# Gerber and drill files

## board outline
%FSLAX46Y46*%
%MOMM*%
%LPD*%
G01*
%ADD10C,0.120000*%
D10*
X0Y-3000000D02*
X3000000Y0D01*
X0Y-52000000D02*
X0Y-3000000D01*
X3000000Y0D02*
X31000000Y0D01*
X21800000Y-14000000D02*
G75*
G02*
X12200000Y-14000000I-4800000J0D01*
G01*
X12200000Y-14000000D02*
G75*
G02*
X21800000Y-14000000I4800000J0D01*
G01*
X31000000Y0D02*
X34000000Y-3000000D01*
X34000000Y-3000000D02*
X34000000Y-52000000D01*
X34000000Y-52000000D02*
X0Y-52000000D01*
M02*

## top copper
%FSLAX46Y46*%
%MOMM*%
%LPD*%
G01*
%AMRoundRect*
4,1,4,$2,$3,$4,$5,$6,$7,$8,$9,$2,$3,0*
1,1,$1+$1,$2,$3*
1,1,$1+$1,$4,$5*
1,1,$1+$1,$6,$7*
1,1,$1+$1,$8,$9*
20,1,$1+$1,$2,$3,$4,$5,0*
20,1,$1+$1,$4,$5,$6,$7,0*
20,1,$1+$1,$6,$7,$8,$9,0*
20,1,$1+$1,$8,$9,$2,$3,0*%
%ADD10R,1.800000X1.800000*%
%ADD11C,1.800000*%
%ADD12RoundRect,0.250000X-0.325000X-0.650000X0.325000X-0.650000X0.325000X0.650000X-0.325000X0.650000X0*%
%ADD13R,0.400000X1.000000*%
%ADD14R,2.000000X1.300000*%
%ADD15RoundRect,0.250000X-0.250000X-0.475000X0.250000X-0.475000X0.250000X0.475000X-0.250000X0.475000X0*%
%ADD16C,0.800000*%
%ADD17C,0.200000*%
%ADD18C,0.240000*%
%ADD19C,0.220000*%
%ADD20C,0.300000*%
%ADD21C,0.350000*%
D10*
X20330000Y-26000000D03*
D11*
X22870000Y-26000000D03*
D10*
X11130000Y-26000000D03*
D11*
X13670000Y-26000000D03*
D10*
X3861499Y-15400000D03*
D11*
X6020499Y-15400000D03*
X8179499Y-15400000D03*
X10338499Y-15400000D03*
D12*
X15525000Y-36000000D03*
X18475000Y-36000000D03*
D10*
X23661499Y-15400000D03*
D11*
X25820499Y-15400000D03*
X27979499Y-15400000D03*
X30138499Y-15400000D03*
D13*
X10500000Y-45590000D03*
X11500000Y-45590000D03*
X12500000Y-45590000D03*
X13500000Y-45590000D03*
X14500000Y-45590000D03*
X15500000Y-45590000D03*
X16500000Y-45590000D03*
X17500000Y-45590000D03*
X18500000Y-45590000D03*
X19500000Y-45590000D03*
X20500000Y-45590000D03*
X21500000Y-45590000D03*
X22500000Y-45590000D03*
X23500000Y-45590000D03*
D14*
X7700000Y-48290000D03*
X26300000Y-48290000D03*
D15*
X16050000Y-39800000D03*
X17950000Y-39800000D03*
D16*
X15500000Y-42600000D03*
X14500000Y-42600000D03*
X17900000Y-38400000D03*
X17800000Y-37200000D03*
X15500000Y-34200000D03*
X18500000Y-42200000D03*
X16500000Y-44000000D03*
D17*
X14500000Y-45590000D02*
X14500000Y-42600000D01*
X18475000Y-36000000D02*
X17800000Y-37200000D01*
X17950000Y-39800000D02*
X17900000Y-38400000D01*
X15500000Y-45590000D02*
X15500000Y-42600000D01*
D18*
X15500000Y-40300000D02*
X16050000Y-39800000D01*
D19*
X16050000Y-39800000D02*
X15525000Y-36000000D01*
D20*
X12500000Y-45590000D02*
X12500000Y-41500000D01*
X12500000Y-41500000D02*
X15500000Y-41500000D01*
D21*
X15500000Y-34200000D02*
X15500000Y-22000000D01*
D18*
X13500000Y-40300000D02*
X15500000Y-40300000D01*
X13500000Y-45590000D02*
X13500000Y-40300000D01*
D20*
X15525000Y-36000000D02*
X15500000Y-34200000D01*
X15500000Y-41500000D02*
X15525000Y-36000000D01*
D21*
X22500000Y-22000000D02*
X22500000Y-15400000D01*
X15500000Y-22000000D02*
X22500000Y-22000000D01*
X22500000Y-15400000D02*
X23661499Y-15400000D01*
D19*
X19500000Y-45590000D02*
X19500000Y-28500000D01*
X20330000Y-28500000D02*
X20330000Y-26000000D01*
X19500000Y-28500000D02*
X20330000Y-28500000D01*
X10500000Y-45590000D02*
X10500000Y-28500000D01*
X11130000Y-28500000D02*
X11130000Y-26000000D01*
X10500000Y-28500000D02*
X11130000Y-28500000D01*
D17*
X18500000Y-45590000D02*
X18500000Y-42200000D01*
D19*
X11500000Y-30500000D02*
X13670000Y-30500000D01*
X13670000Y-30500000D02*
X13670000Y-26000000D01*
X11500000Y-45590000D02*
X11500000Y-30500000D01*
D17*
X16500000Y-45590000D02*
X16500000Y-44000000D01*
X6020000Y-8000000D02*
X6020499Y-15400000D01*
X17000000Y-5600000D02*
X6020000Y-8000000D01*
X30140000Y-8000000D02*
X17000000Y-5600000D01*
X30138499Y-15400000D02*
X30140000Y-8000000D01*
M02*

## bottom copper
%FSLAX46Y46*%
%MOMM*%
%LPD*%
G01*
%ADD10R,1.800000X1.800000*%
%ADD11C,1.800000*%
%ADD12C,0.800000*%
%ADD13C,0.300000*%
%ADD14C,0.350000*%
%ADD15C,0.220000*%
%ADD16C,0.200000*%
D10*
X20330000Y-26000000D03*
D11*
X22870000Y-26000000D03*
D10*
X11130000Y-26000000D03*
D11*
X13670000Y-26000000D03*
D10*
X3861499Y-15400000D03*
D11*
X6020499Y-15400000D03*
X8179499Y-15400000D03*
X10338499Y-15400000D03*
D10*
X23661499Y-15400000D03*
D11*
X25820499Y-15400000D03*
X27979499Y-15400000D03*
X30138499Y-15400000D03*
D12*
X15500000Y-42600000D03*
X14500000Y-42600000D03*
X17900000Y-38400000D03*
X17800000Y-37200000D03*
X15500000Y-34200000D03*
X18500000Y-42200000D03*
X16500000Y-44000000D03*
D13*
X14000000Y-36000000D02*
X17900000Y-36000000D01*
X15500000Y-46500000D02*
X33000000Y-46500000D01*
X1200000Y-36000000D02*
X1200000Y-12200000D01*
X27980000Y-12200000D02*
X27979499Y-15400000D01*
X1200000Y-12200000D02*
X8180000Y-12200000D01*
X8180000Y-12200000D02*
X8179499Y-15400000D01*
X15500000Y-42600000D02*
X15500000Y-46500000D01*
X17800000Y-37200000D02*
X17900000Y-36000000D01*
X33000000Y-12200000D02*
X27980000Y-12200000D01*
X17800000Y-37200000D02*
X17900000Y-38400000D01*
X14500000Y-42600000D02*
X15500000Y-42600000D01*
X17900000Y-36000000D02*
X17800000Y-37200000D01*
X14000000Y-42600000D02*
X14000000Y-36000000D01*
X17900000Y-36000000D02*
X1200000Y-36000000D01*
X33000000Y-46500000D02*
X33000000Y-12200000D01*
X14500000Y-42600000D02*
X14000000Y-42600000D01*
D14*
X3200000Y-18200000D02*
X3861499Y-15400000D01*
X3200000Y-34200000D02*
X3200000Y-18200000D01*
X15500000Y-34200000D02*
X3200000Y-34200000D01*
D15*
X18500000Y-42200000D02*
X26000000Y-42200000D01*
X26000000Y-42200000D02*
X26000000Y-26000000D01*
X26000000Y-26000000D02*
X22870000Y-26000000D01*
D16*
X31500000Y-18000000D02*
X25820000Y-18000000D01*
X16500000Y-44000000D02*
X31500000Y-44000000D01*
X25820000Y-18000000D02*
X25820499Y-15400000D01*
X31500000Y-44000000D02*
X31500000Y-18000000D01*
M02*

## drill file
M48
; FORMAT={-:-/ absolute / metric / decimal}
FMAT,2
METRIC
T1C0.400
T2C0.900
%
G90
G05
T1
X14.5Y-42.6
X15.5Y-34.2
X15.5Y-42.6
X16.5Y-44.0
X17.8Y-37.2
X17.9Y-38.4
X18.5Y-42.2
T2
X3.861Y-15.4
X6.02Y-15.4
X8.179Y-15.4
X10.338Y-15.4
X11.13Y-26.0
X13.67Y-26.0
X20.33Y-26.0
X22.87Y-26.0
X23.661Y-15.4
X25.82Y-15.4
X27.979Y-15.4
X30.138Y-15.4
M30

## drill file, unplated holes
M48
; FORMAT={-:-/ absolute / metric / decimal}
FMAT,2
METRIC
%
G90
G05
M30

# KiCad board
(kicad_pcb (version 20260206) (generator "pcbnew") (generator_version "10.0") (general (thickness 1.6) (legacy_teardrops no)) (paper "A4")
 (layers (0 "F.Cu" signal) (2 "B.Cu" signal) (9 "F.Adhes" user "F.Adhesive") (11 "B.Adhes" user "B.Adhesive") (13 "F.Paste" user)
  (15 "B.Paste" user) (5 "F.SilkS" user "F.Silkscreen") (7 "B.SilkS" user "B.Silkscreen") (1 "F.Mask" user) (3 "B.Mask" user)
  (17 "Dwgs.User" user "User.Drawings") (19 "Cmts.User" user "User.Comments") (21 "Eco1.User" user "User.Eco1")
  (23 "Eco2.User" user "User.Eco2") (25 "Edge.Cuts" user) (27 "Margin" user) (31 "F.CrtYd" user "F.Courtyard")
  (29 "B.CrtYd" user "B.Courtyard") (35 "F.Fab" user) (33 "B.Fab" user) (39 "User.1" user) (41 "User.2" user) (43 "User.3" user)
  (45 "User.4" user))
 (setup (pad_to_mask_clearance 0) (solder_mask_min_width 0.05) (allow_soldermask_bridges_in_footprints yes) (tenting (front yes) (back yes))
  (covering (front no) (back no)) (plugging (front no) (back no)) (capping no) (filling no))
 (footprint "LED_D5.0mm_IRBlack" (layer "F.Cu") (at 20.33 26)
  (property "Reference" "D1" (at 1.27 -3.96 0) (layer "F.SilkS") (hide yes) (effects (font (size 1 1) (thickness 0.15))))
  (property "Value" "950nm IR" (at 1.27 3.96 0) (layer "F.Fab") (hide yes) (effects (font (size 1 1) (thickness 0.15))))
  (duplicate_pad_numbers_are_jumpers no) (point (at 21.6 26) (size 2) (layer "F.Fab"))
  (pad "1" thru_hole rect (at 0 0) (size 1.8 1.8) (drill 0.9) (layers "*.Cu" "*.Mask") (remove_unused_layers no) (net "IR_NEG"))
  (pad "2" thru_hole circle (at 2.54 0) (size 1.8 1.8) (drill 0.9) (layers "*.Cu" "*.Mask") (remove_unused_layers no) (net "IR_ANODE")))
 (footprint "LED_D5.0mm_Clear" (layer "F.Cu") (at 11.13 26)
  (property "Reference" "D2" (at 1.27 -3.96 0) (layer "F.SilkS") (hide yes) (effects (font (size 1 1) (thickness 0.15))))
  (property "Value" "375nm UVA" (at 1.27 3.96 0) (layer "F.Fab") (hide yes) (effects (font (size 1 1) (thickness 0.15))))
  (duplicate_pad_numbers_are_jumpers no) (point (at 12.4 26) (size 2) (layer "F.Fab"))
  (pad "1" thru_hole rect (at 0 0) (size 1.8 1.8) (drill 0.9) (layers "*.Cu" "*.Mask") (remove_unused_layers no) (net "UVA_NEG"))
  (pad "2" thru_hole circle (at 2.54 0) (size 1.8 1.8) (drill 0.9) (layers "*.Cu" "*.Mask") (remove_unused_layers no) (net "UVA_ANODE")))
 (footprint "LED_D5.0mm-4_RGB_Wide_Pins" (layer "F.Cu") (at 3.861499 15.4)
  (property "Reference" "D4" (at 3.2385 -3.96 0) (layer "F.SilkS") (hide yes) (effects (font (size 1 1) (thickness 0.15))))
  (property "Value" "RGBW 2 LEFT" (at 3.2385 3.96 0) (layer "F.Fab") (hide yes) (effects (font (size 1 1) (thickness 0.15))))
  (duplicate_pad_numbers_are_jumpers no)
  (pad "1" thru_hole rect (at 0 0) (size 1.8 1.8) (drill 0.9) (layers "*.Cu" "*.Mask") (remove_unused_layers no) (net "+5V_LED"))
  (pad "2" thru_hole circle (at 2.159 0) (size 1.8 1.8) (drill 0.9) (layers "*.Cu" "*.Mask") (remove_unused_layers no) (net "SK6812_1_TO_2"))
  (pad "3" thru_hole circle (at 4.318 0) (size 1.8 1.8) (drill 0.9) (layers "*.Cu" "*.Mask") (remove_unused_layers no) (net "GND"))
  (pad "4" thru_hole circle (at 6.477 0) (size 1.8 1.8) (drill 0.9) (layers "*.Cu" "*.Mask") (remove_unused_layers no)))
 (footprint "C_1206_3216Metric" (layer "F.Cu") (at 17 36)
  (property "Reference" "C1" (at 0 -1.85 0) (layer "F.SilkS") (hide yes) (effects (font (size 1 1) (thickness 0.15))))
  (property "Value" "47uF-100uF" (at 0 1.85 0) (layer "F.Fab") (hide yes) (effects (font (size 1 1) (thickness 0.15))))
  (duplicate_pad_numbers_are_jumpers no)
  (pad "1" smd roundrect (at -1.475 0) (size 1.15 1.8) (layers "F.Cu" "F.Mask" "F.Paste") (roundrect_rratio 0.217391) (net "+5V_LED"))
  (pad "2" smd roundrect (at 1.475 0) (size 1.15 1.8) (layers "F.Cu" "F.Mask" "F.Paste") (roundrect_rratio 0.217391) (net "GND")))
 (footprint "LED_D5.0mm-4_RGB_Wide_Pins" (layer "F.Cu") (at 23.661499 15.4)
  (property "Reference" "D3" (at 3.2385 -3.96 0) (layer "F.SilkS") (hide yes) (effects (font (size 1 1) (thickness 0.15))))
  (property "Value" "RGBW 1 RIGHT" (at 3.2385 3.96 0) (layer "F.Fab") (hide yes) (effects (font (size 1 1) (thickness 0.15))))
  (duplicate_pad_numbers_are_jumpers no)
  (pad "1" thru_hole rect (at 0 0) (size 1.8 1.8) (drill 0.9) (layers "*.Cu" "*.Mask") (remove_unused_layers no) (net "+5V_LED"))
  (pad "2" thru_hole circle (at 2.159 0) (size 1.8 1.8) (drill 0.9) (layers "*.Cu" "*.Mask") (remove_unused_layers no) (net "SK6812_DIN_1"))
  (pad "3" thru_hole circle (at 4.318 0) (size 1.8 1.8) (drill 0.9) (layers "*.Cu" "*.Mask") (remove_unused_layers no) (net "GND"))
  (pad "4" thru_hole circle (at 6.477 0) (size 1.8 1.8) (drill 0.9) (layers "*.Cu" "*.Mask") (remove_unused_layers no) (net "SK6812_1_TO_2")))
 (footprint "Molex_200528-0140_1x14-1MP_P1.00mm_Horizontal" (layer "F.Cu") (at 17 46.5)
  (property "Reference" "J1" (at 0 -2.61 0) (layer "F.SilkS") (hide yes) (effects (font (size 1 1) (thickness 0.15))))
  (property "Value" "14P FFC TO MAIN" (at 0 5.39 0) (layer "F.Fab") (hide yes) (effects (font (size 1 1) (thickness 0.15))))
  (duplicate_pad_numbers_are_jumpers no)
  (pad "1" smd rect (at -6.5 -0.91) (size 0.4 1) (layers "F.Cu" "F.Mask" "F.Paste") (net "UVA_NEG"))
  (pad "2" smd rect (at -5.5 -0.91) (size 0.4 1) (layers "F.Cu" "F.Mask" "F.Paste") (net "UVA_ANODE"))
  (pad "3" smd rect (at -4.5 -0.91) (size 0.4 1) (layers "F.Cu" "F.Mask" "F.Paste") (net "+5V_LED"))
  (pad "4" smd rect (at -3.5 -0.91) (size 0.4 1) (layers "F.Cu" "F.Mask" "F.Paste") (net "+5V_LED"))
  (pad "5" smd rect (at -2.5 -0.91) (size 0.4 1) (layers "F.Cu" "F.Mask" "F.Paste") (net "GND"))
  (pad "6" smd rect (at -1.5 -0.91) (size 0.4 1) (layers "F.Cu" "F.Mask" "F.Paste") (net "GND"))
  (pad "7" smd rect (at -0.5 -0.91) (size 0.4 1) (layers "F.Cu" "F.Mask" "F.Paste") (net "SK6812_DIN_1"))
  (pad "8" smd rect (at 0.5 -0.91) (size 0.4 1) (layers "F.Cu" "F.Mask" "F.Paste"))
  (pad "9" smd rect (at 1.5 -0.91) (size 0.4 1) (layers "F.Cu" "F.Mask" "F.Paste") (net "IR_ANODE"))
  (pad "10" smd rect (at 2.5 -0.91) (size 0.4 1) (layers "F.Cu" "F.Mask" "F.Paste") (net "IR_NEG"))
  (pad "11" smd rect (at 3.5 -0.91) (size 0.4 1) (layers "F.Cu" "F.Mask" "F.Paste"))
  (pad "12" smd rect (at 4.5 -0.91) (size 0.4 1) (layers "F.Cu" "F.Mask" "F.Paste"))
  (pad "13" smd rect (at 5.5 -0.91) (size 0.4 1) (layers "F.Cu" "F.Mask" "F.Paste"))
  (pad "14" smd rect (at 6.5 -0.91) (size 0.4 1) (layers "F.Cu" "F.Mask" "F.Paste"))
  (pad "MP" smd rect (at -9.3 1.79) (size 2 1.3) (layers "F.Cu" "F.Mask" "F.Paste"))
  (pad "MP" smd rect (at 9.3 1.79) (size 2 1.3) (layers "F.Cu" "F.Mask" "F.Paste")))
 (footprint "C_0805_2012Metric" (layer "F.Cu") (at 17 39.8)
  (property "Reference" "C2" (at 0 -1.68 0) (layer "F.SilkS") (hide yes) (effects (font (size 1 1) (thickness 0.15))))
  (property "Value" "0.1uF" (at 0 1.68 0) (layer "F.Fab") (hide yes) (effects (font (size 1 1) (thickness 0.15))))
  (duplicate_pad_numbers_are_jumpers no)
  (pad "1" smd roundrect (at -0.95 0) (size 1 1.45) (layers "F.Cu" "F.Mask" "F.Paste") (roundrect_rratio 0.25) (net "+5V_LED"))
  (pad "2" smd roundrect (at 0.95 0) (size 1 1.45) (layers "F.Cu" "F.Mask" "F.Paste") (roundrect_rratio 0.25) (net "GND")))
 (gr_line (start 0 3) (end 3 0) (stroke (width 0.12) (type default)) (layer "Edge.Cuts"))
 (gr_line (start 0 52) (end 0 3) (stroke (width 0.12) (type default)) (layer "Edge.Cuts"))
 (gr_line (start 3 0) (end 31 0) (stroke (width 0.12) (type default)) (layer "Edge.Cuts"))
 (gr_circle (center 17 14) (end 21.8 14) (stroke (width 0.12) (type default)) (fill no) (layer "Edge.Cuts"))
 (gr_line (start 31 0) (end 34 3) (stroke (width 0.12) (type default)) (layer "Edge.Cuts"))
 (gr_line (start 34 3) (end 34 52) (stroke (width 0.12) (type default)) (layer "Edge.Cuts"))
 (gr_line (start 34 52) (end 0 52) (stroke (width 0.12) (type default)) (layer "Edge.Cuts"))
 (segment (start 14.5 45.59) (end 14.5 42.6) (width 0.2) (layer "F.Cu") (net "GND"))
 (segment (start 18.475 36) (end 17.8 37.2) (width 0.2) (layer "F.Cu") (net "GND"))
 (segment (start 17.95 39.8) (end 17.9 38.4) (width 0.2) (layer "F.Cu") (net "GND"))
 (segment (start 15.5 45.59) (end 15.5 42.6) (width 0.2) (layer "F.Cu") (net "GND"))
 (via (at 15.5 42.6) (size 0.8) (drill 0.4) (layers "F.Cu" "B.Cu") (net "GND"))
 (via (at 14.5 42.6) (size 0.8) (drill 0.4) (layers "F.Cu" "B.Cu") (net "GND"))
 (via (at 17.9 38.4) (size 0.8) (drill 0.4) (layers "F.Cu" "B.Cu") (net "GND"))
 (via (at 17.8 37.2) (size 0.8) (drill 0.4) (layers "F.Cu" "B.Cu") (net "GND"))
 (segment (start 14 36) (end 17.9 36) (width 0.3) (layer "B.Cu") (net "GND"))
 (segment (start 15.5 46.5) (end 33 46.5) (width 0.3) (layer "B.Cu") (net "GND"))
 (segment (start 1.2 36) (end 1.2 12.2) (width 0.3) (layer "B.Cu") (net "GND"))
 (segment (start 27.98 12.2) (end 27.979499 15.4) (width 0.3) (layer "B.Cu") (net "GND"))
 (segment (start 1.2 12.2) (end 8.18 12.2) (width 0.3) (layer "B.Cu") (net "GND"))
 (segment (start 8.18 12.2) (end 8.179499 15.4) (width 0.3) (layer "B.Cu") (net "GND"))
 (segment (start 15.5 42.6) (end 15.5 46.5) (width 0.3) (layer "B.Cu") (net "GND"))
 (segment (start 17.8 37.2) (end 17.9 36) (width 0.3) (layer "B.Cu") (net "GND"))
 (segment (start 33 12.2) (end 27.98 12.2) (width 0.3) (layer "B.Cu") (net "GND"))
 (segment (start 17.8 37.2) (end 17.9 38.4) (width 0.3) (layer "B.Cu") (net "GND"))
 (segment (start 14.5 42.6) (end 15.5 42.6) (width 0.3) (layer "B.Cu") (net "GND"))
 (segment (start 17.9 36) (end 17.8 37.2) (width 0.3) (layer "B.Cu") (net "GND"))
 (segment (start 14 42.6) (end 14 36) (width 0.3) (layer "B.Cu") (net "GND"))
 (segment (start 17.9 36) (end 1.2 36) (width 0.3) (layer "B.Cu") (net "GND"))
 (segment (start 33 46.5) (end 33 12.2) (width 0.3) (layer "B.Cu") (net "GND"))
 (segment (start 14.5 42.6) (end 14 42.6) (width 0.3) (layer "B.Cu") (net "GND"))
 (segment (start 15.5 40.3) (end 16.05 39.8) (width 0.24) (layer "F.Cu") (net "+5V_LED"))
 (segment (start 16.05 39.8) (end 15.525 36) (width 0.22) (layer "F.Cu") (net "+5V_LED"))
 (segment (start 12.5 45.59) (end 12.5 41.5) (width 0.3) (layer "F.Cu") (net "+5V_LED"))
 (segment (start 12.5 41.5) (end 15.5 41.5) (width 0.3) (layer "F.Cu") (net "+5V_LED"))
 (segment (start 15.5 34.2) (end 15.5 22) (width 0.35) (layer "F.Cu") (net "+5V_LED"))
 (segment (start 13.5 40.3) (end 15.5 40.3) (width 0.24) (layer "F.Cu") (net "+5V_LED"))
 (segment (start 13.5 45.59) (end 13.5 40.3) (width 0.24) (layer "F.Cu") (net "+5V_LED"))
 (segment (start 15.525 36) (end 15.5 34.2) (width 0.3) (layer "F.Cu") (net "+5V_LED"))
 (segment (start 15.5 41.5) (end 15.525 36) (width 0.3) (layer "F.Cu") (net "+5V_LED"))
 (segment (start 22.5 22) (end 22.5 15.4) (width 0.35) (layer "F.Cu") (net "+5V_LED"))
 (segment (start 15.5 22) (end 22.5 22) (width 0.35) (layer "F.Cu") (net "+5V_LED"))
 (segment (start 22.5 15.4) (end 23.661499 15.4) (width 0.35) (layer "F.Cu") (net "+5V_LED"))
 (via (at 15.5 34.2) (size 0.8) (drill 0.4) (layers "F.Cu" "B.Cu") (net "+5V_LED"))
 (segment (start 3.2 18.2) (end 3.861499 15.4) (width 0.35) (layer "B.Cu") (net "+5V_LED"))
 (segment (start 3.2 34.2) (end 3.2 18.2) (width 0.35) (layer "B.Cu") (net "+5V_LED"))
 (segment (start 15.5 34.2) (end 3.2 34.2) (width 0.35) (layer "B.Cu") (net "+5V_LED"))
 (segment (start 19.5 45.59) (end 19.5 28.5) (width 0.22) (layer "F.Cu") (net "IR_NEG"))
 (segment (start 20.33 28.5) (end 20.33 26) (width 0.22) (layer "F.Cu") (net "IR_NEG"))
 (segment (start 19.5 28.5) (end 20.33 28.5) (width 0.22) (layer "F.Cu") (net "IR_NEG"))
 (segment (start 10.5 45.59) (end 10.5 28.5) (width 0.22) (layer "F.Cu") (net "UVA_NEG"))
 (segment (start 11.13 28.5) (end 11.13 26) (width 0.22) (layer "F.Cu") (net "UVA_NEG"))
 (segment (start 10.5 28.5) (end 11.13 28.5) (width 0.22) (layer "F.Cu") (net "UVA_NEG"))
 (segment (start 18.5 45.59) (end 18.5 42.2) (width 0.2) (layer "F.Cu") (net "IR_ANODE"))
 (via (at 18.5 42.2) (size 0.8) (drill 0.4) (layers "F.Cu" "B.Cu") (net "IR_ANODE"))
 (segment (start 18.5 42.2) (end 26 42.2) (width 0.22) (layer "B.Cu") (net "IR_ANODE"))
 (segment (start 26 42.2) (end 26 26) (width 0.22) (layer "B.Cu") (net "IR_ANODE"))
 (segment (start 26 26) (end 22.87 26) (width 0.22) (layer "B.Cu") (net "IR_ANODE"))
 (segment (start 11.5 30.5) (end 13.67 30.5) (width 0.22) (layer "F.Cu") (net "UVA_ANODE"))
 (segment (start 13.67 30.5) (end 13.67 26) (width 0.22) (layer "F.Cu") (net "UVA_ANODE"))
 (segment (start 11.5 45.59) (end 11.5 30.5) (width 0.22) (layer "F.Cu") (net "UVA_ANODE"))
 (segment (start 16.5 45.59) (end 16.5 44) (width 0.2) (layer "F.Cu") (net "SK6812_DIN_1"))
 (via (at 16.5 44) (size 0.8) (drill 0.4) (layers "F.Cu" "B.Cu") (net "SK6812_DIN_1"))
 (segment (start 31.5 18) (end 25.82 18) (width 0.2) (layer "B.Cu") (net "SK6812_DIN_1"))
 (segment (start 16.5 44) (end 31.5 44) (width 0.2) (layer "B.Cu") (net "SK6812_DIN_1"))
 (segment (start 25.82 18) (end 25.820499 15.4) (width 0.2) (layer "B.Cu") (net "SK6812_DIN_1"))
 (segment (start 31.5 44) (end 31.5 18) (width 0.2) (layer "B.Cu") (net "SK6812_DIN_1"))
 (segment (start 6.02 8) (end 6.020499 15.4) (width 0.2) (layer "F.Cu") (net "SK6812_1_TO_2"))
 (segment (start 17 5.6) (end 6.02 8) (width 0.2) (layer "F.Cu") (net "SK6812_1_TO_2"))
 (segment (start 30.14 8) (end 17 5.6) (width 0.2) (layer "F.Cu") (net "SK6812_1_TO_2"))
 (segment (start 30.138499 15.4) (end 30.14 8) (width 0.2) (layer "F.Cu") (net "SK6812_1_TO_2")))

